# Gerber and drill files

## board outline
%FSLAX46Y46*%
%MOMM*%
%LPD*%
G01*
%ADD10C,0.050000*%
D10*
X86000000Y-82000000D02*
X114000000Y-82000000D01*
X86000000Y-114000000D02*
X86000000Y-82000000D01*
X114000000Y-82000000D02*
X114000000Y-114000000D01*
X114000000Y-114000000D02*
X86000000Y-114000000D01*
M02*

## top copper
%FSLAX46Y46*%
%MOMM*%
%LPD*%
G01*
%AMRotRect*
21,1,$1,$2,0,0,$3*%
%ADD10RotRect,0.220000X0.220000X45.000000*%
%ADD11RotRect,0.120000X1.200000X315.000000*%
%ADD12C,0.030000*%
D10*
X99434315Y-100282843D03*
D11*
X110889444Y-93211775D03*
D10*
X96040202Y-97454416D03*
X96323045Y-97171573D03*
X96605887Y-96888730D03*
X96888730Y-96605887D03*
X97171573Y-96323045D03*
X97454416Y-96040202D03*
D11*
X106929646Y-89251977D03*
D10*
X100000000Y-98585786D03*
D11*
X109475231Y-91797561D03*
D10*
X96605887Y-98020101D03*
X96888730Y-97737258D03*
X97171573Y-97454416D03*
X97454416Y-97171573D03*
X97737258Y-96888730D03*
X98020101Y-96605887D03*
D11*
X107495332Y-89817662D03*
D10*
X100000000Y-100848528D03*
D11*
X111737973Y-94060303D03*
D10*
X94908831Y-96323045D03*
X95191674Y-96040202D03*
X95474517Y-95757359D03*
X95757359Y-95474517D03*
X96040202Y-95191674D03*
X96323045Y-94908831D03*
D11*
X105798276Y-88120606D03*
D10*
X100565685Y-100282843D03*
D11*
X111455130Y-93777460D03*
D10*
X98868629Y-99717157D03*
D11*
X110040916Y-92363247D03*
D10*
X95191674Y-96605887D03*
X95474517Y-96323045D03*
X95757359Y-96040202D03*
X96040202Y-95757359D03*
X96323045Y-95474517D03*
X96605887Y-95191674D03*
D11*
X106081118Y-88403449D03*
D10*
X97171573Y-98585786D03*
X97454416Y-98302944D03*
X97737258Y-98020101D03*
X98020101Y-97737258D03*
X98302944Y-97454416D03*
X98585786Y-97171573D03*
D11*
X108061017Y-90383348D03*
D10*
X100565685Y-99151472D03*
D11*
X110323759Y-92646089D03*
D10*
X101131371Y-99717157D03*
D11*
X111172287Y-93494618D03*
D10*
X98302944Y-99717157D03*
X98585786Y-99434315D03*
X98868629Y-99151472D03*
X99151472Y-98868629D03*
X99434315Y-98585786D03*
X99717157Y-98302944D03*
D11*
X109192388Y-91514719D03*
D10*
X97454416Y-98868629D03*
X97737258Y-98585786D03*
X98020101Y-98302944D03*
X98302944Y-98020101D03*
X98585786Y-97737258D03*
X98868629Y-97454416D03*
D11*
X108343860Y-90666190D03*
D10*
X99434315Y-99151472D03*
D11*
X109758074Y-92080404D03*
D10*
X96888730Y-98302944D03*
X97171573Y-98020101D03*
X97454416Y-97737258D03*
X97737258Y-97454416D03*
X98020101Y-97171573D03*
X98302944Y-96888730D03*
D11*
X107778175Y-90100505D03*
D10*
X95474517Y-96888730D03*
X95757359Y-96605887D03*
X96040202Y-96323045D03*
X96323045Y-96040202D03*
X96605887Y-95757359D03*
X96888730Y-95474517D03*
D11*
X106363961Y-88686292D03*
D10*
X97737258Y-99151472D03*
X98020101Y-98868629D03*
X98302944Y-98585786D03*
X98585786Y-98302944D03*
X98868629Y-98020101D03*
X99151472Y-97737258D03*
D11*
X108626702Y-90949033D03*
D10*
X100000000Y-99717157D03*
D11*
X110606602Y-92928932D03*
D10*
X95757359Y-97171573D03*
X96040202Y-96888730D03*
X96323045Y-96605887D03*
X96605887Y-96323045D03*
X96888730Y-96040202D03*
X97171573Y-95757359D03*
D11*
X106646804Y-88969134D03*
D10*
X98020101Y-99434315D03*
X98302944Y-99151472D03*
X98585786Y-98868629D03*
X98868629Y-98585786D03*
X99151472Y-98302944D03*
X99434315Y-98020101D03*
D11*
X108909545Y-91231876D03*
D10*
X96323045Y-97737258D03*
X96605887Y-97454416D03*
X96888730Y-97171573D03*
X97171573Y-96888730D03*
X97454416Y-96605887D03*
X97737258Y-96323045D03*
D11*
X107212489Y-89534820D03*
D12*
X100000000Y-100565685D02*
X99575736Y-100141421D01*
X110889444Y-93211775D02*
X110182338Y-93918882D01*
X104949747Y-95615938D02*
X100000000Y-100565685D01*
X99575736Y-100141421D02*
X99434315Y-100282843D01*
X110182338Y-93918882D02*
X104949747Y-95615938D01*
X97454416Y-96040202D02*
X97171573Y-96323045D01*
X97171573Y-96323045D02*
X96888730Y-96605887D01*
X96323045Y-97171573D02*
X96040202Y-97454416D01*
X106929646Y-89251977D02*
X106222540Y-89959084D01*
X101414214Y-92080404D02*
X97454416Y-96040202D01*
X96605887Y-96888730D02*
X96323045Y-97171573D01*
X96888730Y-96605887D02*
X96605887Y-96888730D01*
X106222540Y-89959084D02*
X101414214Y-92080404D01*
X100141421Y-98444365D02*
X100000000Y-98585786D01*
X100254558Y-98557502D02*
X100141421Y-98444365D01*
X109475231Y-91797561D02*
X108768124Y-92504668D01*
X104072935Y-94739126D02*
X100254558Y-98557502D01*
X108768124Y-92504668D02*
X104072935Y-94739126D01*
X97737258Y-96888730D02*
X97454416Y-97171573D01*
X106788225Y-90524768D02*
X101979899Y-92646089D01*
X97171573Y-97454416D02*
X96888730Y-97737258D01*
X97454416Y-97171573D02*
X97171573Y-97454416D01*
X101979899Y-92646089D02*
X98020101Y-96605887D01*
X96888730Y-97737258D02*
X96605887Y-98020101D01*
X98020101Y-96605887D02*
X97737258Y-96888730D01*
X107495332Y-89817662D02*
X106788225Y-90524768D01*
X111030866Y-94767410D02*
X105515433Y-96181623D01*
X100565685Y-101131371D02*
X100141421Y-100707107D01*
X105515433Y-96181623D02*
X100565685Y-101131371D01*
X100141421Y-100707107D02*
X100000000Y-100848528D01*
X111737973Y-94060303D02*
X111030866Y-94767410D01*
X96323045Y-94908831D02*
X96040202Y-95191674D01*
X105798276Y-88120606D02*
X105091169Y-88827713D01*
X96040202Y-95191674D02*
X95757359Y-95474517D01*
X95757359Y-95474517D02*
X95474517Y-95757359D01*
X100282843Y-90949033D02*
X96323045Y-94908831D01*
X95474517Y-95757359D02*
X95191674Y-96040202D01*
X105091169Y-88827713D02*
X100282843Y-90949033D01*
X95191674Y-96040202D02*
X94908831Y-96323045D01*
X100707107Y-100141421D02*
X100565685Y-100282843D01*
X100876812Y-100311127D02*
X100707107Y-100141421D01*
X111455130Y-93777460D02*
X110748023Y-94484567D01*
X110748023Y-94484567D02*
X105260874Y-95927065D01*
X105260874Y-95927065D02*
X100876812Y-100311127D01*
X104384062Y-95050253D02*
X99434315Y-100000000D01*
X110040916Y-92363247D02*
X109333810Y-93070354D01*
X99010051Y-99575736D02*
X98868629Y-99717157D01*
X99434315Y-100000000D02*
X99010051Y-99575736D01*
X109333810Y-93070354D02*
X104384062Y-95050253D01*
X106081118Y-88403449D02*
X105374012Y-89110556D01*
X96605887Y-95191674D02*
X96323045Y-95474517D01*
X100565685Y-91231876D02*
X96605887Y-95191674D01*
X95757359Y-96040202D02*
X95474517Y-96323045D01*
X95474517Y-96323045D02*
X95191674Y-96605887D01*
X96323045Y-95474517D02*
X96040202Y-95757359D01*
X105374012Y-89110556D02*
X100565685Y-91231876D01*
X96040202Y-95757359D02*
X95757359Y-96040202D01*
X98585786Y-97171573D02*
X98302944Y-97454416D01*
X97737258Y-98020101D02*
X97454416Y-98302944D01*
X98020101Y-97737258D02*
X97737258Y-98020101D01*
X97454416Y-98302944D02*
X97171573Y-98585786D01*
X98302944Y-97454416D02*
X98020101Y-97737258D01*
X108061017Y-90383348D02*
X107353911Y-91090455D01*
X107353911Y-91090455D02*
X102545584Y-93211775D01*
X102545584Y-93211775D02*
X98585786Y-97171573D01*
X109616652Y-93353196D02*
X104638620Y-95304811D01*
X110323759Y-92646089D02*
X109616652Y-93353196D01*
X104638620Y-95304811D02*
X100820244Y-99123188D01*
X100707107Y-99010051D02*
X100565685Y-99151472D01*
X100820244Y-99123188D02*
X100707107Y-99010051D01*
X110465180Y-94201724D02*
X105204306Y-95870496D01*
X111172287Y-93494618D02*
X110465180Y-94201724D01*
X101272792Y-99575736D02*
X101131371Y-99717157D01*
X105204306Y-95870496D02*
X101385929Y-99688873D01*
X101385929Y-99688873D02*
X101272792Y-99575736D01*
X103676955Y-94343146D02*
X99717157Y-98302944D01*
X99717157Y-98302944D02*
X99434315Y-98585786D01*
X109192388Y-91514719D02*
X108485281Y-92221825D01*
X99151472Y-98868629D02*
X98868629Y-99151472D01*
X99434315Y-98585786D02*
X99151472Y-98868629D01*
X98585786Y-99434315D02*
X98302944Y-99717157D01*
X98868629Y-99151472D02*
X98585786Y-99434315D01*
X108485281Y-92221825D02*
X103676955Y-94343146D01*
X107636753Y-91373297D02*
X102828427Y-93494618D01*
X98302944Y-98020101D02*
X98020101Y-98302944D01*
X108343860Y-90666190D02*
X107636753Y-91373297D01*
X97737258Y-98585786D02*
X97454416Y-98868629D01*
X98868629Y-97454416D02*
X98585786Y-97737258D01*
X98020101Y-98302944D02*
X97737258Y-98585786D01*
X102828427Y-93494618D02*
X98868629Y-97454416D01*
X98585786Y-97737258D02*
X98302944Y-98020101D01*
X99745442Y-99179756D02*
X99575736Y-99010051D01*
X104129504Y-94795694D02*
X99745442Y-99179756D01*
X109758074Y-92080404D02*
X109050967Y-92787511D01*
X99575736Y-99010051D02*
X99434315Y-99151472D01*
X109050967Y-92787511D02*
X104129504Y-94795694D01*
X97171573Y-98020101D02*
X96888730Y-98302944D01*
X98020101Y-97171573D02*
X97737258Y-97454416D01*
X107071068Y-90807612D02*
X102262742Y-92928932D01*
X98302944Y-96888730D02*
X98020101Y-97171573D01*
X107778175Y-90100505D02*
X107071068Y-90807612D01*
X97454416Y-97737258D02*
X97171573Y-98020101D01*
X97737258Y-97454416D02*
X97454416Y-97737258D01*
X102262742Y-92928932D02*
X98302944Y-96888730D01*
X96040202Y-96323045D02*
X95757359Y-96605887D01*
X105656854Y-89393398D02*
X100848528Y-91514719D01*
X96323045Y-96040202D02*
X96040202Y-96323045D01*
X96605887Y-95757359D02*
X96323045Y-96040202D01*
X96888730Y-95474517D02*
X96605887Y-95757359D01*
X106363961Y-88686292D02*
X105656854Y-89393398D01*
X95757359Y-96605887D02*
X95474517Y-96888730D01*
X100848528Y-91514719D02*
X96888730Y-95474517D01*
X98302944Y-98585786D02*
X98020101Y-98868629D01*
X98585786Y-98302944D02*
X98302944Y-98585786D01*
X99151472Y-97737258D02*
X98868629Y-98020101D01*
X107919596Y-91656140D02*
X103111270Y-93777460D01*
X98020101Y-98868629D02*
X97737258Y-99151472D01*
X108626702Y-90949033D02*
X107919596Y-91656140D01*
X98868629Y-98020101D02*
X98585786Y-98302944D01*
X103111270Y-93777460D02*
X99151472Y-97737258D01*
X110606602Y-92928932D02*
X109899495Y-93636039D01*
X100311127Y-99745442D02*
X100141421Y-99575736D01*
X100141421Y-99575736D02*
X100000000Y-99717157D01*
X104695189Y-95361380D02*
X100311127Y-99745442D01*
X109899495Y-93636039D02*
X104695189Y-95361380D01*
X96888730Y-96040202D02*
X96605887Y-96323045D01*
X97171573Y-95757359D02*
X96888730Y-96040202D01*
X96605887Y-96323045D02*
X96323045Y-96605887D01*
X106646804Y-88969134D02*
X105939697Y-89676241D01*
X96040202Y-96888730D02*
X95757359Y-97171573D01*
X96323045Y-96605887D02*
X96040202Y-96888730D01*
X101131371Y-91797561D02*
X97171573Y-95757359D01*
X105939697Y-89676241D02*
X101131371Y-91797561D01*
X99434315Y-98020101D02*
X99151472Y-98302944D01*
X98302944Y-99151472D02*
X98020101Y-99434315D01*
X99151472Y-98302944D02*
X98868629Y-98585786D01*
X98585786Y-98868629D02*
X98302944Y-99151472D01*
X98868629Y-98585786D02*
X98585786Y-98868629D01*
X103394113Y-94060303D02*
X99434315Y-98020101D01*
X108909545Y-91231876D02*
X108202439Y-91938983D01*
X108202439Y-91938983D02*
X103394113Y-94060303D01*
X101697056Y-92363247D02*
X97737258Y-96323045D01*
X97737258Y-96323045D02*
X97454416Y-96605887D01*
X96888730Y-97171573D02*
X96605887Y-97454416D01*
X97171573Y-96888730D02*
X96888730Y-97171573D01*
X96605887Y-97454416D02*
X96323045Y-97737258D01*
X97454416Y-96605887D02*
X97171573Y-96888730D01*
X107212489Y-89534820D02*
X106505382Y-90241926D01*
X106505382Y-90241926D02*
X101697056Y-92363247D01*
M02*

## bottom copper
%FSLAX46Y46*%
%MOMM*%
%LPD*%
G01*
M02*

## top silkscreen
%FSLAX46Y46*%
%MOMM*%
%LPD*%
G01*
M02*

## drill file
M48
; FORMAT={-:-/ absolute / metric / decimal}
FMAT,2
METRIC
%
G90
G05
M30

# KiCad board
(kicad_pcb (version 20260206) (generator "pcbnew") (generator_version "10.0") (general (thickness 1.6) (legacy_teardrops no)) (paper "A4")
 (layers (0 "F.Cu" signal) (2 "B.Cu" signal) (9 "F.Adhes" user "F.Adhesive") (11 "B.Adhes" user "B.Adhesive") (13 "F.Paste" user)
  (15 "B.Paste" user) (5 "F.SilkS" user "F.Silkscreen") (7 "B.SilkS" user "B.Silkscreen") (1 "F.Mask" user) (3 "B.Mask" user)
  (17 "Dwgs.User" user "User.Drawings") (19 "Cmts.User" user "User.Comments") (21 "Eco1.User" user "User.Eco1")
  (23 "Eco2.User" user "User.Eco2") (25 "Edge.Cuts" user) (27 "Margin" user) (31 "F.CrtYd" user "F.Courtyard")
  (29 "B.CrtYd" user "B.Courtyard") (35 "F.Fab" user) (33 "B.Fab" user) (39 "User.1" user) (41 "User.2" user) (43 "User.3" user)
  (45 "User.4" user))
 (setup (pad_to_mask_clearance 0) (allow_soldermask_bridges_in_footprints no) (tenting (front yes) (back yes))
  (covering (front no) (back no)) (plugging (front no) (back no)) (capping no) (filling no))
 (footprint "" (layer "F.Cu") (at 0 0)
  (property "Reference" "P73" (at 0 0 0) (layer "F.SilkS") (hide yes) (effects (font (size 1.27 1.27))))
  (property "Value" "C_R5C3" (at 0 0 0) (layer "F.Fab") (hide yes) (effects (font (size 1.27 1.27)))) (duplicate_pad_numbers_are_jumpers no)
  (pad "1" connect rect (at 99.434315 100.282843 45) (size 0.22 0.22) (layers "F.Cu") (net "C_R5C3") (thermal_bridge_angle 45))
  (pad "2" connect rect (at 110.889444 93.211775 315) (size 0.12 1.2) (layers "F.Cu") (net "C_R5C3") (thermal_bridge_angle 45)))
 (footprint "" (layer "F.Cu") (at 0 0)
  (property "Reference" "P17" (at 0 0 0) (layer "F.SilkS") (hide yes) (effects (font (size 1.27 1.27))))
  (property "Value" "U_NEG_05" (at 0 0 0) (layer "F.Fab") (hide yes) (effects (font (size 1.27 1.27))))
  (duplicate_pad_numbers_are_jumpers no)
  (pad "1" connect rect (at 96.040202 97.454416 45) (size 0.22 0.22) (layers "F.Cu") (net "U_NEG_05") (thermal_bridge_angle 45))
  (pad "1" connect rect (at 96.323045 97.171573 45) (size 0.22 0.22) (layers "F.Cu") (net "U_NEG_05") (thermal_bridge_angle 45))
  (pad "1" connect rect (at 96.605887 96.88873 45) (size 0.22 0.22) (layers "F.Cu") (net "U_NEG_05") (thermal_bridge_angle 45))
  (pad "1" connect rect (at 96.88873 96.605887 45) (size 0.22 0.22) (layers "F.Cu") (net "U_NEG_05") (thermal_bridge_angle 45))
  (pad "1" connect rect (at 97.171573 96.323045 45) (size 0.22 0.22) (layers "F.Cu") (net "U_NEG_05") (thermal_bridge_angle 45))
  (pad "1" connect rect (at 97.454416 96.040202 45) (size 0.22 0.22) (layers "F.Cu") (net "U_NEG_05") (thermal_bridge_angle 45))
  (pad "2" connect rect (at 106.929646 89.251977 315) (size 0.12 1.2) (layers "F.Cu") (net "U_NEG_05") (thermal_bridge_angle 45)))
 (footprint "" (layer "F.Cu") (at 0 0)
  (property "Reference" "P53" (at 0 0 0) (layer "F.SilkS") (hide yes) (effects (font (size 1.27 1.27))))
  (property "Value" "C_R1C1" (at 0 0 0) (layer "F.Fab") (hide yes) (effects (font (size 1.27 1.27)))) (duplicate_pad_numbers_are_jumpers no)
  (pad "1" connect rect (at 100 98.585786 45) (size 0.22 0.22) (layers "F.Cu") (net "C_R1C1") (thermal_bridge_angle 45))
  (pad "2" connect rect (at 109.475231 91.797561 315) (size 0.12 1.2) (layers "F.Cu") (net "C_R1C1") (thermal_bridge_angle 45)))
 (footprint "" (layer "F.Cu") (at 0 0)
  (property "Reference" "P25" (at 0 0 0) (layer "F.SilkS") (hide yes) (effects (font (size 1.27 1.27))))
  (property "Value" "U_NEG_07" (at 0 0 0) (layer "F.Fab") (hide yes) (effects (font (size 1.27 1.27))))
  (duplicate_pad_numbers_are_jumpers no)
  (pad "1" connect rect (at 96.605887 98.020101 45) (size 0.22 0.22) (layers "F.Cu") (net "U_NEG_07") (thermal_bridge_angle 45))
  (pad "1" connect rect (at 96.88873 97.737258 45) (size 0.22 0.22) (layers "F.Cu") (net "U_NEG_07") (thermal_bridge_angle 45))
  (pad "1" connect rect (at 97.171573 97.454416 45) (size 0.22 0.22) (layers "F.Cu") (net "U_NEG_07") (thermal_bridge_angle 45))
  (pad "1" connect rect (at 97.454416 97.171573 45) (size 0.22 0.22) (layers "F.Cu") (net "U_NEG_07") (thermal_bridge_angle 45))
  (pad "1" connect rect (at 97.737258 96.88873 45) (size 0.22 0.22) (layers "F.Cu") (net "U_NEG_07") (thermal_bridge_angle 45))
  (pad "1" connect rect (at 98.020101 96.605887 45) (size 0.22 0.22) (layers "F.Cu") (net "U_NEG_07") (thermal_bridge_angle 45))
  (pad "2" connect rect (at 107.495332 89.817662 315) (size 0.12 1.2) (layers "F.Cu") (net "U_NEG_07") (thermal_bridge_angle 45)))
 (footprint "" (layer "F.Cu") (at 0 0)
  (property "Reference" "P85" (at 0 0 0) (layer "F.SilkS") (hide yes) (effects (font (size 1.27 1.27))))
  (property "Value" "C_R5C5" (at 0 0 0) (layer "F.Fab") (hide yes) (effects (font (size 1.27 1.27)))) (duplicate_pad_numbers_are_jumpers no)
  (pad "1" connect rect (at 100 100.848528 45) (size 0.22 0.22) (layers "F.Cu") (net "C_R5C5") (thermal_bridge_angle 45))
  (pad "2" connect rect (at 111.737973 94.060303 315) (size 0.12 1.2) (layers "F.Cu") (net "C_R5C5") (thermal_bridge_angle 45)))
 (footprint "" (layer "F.Cu") (at 0 0)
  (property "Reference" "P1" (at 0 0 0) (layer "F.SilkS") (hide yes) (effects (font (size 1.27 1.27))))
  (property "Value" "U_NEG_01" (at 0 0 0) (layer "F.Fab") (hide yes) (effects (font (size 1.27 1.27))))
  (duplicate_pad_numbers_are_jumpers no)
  (pad "1" connect rect (at 94.908831 96.323045 45) (size 0.22 0.22) (layers "F.Cu") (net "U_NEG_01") (thermal_bridge_angle 45))
  (pad "1" connect rect (at 95.191674 96.040202 45) (size 0.22 0.22) (layers "F.Cu") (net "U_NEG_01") (thermal_bridge_angle 45))
  (pad "1" connect rect (at 95.474517 95.757359 45) (size 0.22 0.22) (layers "F.Cu") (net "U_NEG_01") (thermal_bridge_angle 45))
  (pad "1" connect rect (at 95.757359 95.474517 45) (size 0.22 0.22) (layers "F.Cu") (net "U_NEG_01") (thermal_bridge_angle 45))
  (pad "1" connect rect (at 96.040202 95.191674 45) (size 0.22 0.22) (layers "F.Cu") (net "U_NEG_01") (thermal_bridge_angle 45))
  (pad "1" connect rect (at 96.323045 94.908831 45) (size 0.22 0.22) (layers "F.Cu") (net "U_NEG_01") (thermal_bridge_angle 45))
  (pad "2" connect rect (at 105.798276 88.120606 315) (size 0.12 1.2) (layers "F.Cu") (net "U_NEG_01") (thermal_bridge_angle 45)))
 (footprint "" (layer "F.Cu") (at 0 0)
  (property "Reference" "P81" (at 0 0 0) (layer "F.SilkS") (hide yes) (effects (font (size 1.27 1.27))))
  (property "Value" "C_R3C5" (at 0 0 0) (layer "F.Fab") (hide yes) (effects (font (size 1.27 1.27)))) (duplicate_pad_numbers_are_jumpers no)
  (pad "1" connect rect (at 100.565685 100.282843 45) (size 0.22 0.22) (layers "F.Cu") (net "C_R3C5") (thermal_bridge_angle 45))
  (pad "2" connect rect (at 111.45513 93.77746 315) (size 0.12 1.2) (layers "F.Cu") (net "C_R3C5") (thermal_bridge_angle 45)))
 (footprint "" (layer "F.Cu") (at 0 0)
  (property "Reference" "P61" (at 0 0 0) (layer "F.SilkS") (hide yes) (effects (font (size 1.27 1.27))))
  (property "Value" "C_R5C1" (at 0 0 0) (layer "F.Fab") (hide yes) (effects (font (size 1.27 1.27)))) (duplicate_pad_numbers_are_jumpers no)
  (pad "1" connect rect (at 98.868629 99.717157 45) (size 0.22 0.22) (layers "F.Cu") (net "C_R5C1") (thermal_bridge_angle 45))
  (pad "2" connect rect (at 110.040916 92.363247 315) (size 0.12 1.2) (layers "F.Cu") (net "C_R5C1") (thermal_bridge_angle 45)))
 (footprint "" (layer "F.Cu") (at 0 0)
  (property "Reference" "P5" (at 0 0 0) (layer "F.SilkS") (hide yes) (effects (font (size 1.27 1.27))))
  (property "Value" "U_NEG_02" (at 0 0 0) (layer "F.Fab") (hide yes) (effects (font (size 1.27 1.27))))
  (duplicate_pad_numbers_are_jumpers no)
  (pad "1" connect rect (at 95.191674 96.605887 45) (size 0.22 0.22) (layers "F.Cu") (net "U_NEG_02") (thermal_bridge_angle 45))
  (pad "1" connect rect (at 95.474517 96.323045 45) (size 0.22 0.22) (layers "F.Cu") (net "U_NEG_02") (thermal_bridge_angle 45))
  (pad "1" connect rect (at 95.757359 96.040202 45) (size 0.22 0.22) (layers "F.Cu") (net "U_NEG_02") (thermal_bridge_angle 45))
  (pad "1" connect rect (at 96.040202 95.757359 45) (size 0.22 0.22) (layers "F.Cu") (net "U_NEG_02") (thermal_bridge_angle 45))
  (pad "1" connect rect (at 96.323045 95.474517 45) (size 0.22 0.22) (layers "F.Cu") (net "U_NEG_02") (thermal_bridge_angle 45))
  (pad "1" connect rect (at 96.605887 95.191674 45) (size 0.22 0.22) (layers "F.Cu") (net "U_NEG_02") (thermal_bridge_angle 45))
  (pad "2" connect rect (at 106.081118 88.403449 315) (size 0.12 1.2) (layers "F.Cu") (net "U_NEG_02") (thermal_bridge_angle 45)))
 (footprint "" (layer "F.Cu") (at 0 0)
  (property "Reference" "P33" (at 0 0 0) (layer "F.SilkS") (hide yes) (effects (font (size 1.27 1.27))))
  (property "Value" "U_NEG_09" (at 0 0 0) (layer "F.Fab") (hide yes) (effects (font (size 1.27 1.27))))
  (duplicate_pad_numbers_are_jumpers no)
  (pad "1" connect rect (at 97.171573 98.585786 45) (size 0.22 0.22) (layers "F.Cu") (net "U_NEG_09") (thermal_bridge_angle 45))
  (pad "1" connect rect (at 97.454416 98.302944 45) (size 0.22 0.22) (layers "F.Cu") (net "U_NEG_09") (thermal_bridge_angle 45))
  (pad "1" connect rect (at 97.737258 98.020101 45) (size 0.22 0.22) (layers "F.Cu") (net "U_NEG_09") (thermal_bridge_angle 45))
  (pad "1" connect rect (at 98.020101 97.737258 45) (size 0.22 0.22) (layers "F.Cu") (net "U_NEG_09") (thermal_bridge_angle 45))
  (pad "1" connect rect (at 98.302944 97.454416 45) (size 0.22 0.22) (layers "F.Cu") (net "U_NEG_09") (thermal_bridge_angle 45))
  (pad "1" connect rect (at 98.585786 97.171573 45) (size 0.22 0.22) (layers "F.Cu") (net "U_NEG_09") (thermal_bridge_angle 45))
  (pad "2" connect rect (at 108.061017 90.383348 315) (size 0.12 1.2) (layers "F.Cu") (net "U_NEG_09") (thermal_bridge_angle 45)))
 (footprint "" (layer "F.Cu") (at 0 0)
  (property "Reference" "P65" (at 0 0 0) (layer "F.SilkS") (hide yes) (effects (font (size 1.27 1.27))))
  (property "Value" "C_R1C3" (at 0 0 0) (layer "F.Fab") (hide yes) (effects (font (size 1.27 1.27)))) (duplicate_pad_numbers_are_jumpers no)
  (pad "1" connect rect (at 100.565685 99.151472 45) (size 0.22 0.22) (layers "F.Cu") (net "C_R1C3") (thermal_bridge_angle 45))
  (pad "2" connect rect (at 110.323759 92.646089 315) (size 0.12 1.2) (layers "F.Cu") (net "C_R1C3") (thermal_bridge_angle 45)))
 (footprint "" (layer "F.Cu") (at 0 0)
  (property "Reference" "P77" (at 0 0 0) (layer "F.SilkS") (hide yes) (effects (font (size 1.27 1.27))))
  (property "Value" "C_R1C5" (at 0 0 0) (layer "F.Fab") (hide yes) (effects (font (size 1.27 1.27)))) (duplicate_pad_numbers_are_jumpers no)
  (pad "1" connect rect (at 101.131371 99.717157 45) (size 0.22 0.22) (layers "F.Cu") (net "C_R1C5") (thermal_bridge_angle 45))
  (pad "2" connect rect (at 111.172287 93.494618 315) (size 0.12 1.2) (layers "F.Cu") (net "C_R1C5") (thermal_bridge_angle 45)))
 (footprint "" (layer "F.Cu") (at 0 0)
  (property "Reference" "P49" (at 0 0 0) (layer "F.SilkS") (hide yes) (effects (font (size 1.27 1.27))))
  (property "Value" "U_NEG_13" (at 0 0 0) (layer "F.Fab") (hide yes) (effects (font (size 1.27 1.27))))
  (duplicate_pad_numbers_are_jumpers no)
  (pad "1" connect rect (at 98.302944 99.717157 45) (size 0.22 0.22) (layers "F.Cu") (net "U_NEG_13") (thermal_bridge_angle 45))
  (pad "1" connect rect (at 98.585786 99.434315 45) (size 0.22 0.22) (layers "F.Cu") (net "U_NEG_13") (thermal_bridge_angle 45))
  (pad "1" connect rect (at 98.868629 99.151472 45) (size 0.22 0.22) (layers "F.Cu") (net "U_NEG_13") (thermal_bridge_angle 45))
  (pad "1" connect rect (at 99.151472 98.868629 45) (size 0.22 0.22) (layers "F.Cu") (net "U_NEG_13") (thermal_bridge_angle 45))
  (pad "1" connect rect (at 99.434315 98.585786 45) (size 0.22 0.22) (layers "F.Cu") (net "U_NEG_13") (thermal_bridge_angle 45))
  (pad "1" connect rect (at 99.717157 98.302944 45) (size 0.22 0.22) (layers "F.Cu") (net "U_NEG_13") (thermal_bridge_angle 45))
  (pad "2" connect rect (at 109.192388 91.514719 315) (size 0.12 1.2) (layers "F.Cu") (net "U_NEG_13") (thermal_bridge_angle 45)))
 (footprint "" (layer "F.Cu") (at 0 0)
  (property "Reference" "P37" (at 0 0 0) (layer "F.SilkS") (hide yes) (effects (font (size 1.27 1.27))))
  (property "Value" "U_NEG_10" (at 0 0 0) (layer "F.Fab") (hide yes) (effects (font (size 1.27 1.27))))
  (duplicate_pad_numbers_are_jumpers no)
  (pad "1" connect rect (at 97.454416 98.868629 45) (size 0.22 0.22) (layers "F.Cu") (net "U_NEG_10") (thermal_bridge_angle 45))
  (pad "1" connect rect (at 97.737258 98.585786 45) (size 0.22 0.22) (layers "F.Cu") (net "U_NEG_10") (thermal_bridge_angle 45))
  (pad "1" connect rect (at 98.020101 98.302944 45) (size 0.22 0.22) (layers "F.Cu") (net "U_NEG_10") (thermal_bridge_angle 45))
  (pad "1" connect rect (at 98.302944 98.020101 45) (size 0.22 0.22) (layers "F.Cu") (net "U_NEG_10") (thermal_bridge_angle 45))
  (pad "1" connect rect (at 98.585786 97.737258 45) (size 0.22 0.22) (layers "F.Cu") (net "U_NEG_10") (thermal_bridge_angle 45))
  (pad "1" connect rect (at 98.868629 97.454416 45) (size 0.22 0.22) (layers "F.Cu") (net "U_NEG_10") (thermal_bridge_angle 45))
  (pad "2" connect rect (at 108.34386 90.66619 315) (size 0.12 1.2) (layers "F.Cu") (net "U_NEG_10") (thermal_bridge_angle 45)))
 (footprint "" (layer "F.Cu") (at 0 0)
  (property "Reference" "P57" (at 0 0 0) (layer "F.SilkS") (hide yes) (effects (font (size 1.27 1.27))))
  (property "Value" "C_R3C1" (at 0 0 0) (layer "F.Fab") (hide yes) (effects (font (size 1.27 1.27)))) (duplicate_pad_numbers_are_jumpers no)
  (pad "1" connect rect (at 99.434315 99.151472 45) (size 0.22 0.22) (layers "F.Cu") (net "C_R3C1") (thermal_bridge_angle 45))
  (pad "2" connect rect (at 109.758074 92.080404 315) (size 0.12 1.2) (layers "F.Cu") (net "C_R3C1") (thermal_bridge_angle 45)))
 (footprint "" (layer "F.Cu") (at 0 0)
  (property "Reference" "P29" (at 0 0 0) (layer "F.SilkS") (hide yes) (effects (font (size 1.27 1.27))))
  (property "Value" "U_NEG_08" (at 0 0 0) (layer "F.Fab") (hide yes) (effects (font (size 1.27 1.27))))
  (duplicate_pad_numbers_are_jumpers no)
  (pad "1" connect rect (at 96.88873 98.302944 45) (size 0.22 0.22) (layers "F.Cu") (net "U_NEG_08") (thermal_bridge_angle 45))
  (pad "1" connect rect (at 97.171573 98.020101 45) (size 0.22 0.22) (layers "F.Cu") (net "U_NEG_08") (thermal_bridge_angle 45))
  (pad "1" connect rect (at 97.454416 97.737258 45) (size 0.22 0.22) (layers "F.Cu") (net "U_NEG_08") (thermal_bridge_angle 45))
  (pad "1" connect rect (at 97.737258 97.454416 45) (size 0.22 0.22) (layers "F.Cu") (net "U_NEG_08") (thermal_bridge_angle 45))
  (pad "1" connect rect (at 98.020101 97.171573 45) (size 0.22 0.22) (layers "F.Cu") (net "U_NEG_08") (thermal_bridge_angle 45))
  (pad "1" connect rect (at 98.302944 96.88873 45) (size 0.22 0.22) (layers "F.Cu") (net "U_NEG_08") (thermal_bridge_angle 45))
  (pad "2" connect rect (at 107.778175 90.100505 315) (size 0.12 1.2) (layers "F.Cu") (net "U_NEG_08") (thermal_bridge_angle 45)))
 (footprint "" (layer "F.Cu") (at 0 0)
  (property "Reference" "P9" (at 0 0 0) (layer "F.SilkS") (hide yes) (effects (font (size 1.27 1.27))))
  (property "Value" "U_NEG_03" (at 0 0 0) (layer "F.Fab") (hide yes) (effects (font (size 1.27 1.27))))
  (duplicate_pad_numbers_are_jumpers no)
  (pad "1" connect rect (at 95.474517 96.88873 45) (size 0.22 0.22) (layers "F.Cu") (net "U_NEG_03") (thermal_bridge_angle 45))
  (pad "1" connect rect (at 95.757359 96.605887 45) (size 0.22 0.22) (layers "F.Cu") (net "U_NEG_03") (thermal_bridge_angle 45))
  (pad "1" connect rect (at 96.040202 96.323045 45) (size 0.22 0.22) (layers "F.Cu") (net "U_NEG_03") (thermal_bridge_angle 45))
  (pad "1" connect rect (at 96.323045 96.040202 45) (size 0.22 0.22) (layers "F.Cu") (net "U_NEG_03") (thermal_bridge_angle 45))
  (pad "1" connect rect (at 96.605887 95.757359 45) (size 0.22 0.22) (layers "F.Cu") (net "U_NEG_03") (thermal_bridge_angle 45))
  (pad "1" connect rect (at 96.88873 95.474517 45) (size 0.22 0.22) (layers "F.Cu") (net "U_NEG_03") (thermal_bridge_angle 45))
  (pad "2" connect rect (at 106.363961 88.686292 315) (size 0.12 1.2) (layers "F.Cu") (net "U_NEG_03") (thermal_bridge_angle 45)))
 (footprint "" (layer "F.Cu") (at 0 0)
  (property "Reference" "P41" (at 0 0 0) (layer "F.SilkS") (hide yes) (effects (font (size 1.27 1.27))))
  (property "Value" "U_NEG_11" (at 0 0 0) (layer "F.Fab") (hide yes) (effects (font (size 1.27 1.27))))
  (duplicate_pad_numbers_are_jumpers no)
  (pad "1" connect rect (at 97.737258 99.151472 45) (size 0.22 0.22) (layers "F.Cu") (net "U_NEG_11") (thermal_bridge_angle 45))
  (pad "1" connect rect (at 98.020101 98.868629 45) (size 0.22 0.22) (layers "F.Cu") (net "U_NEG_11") (thermal_bridge_angle 45))
  (pad "1" connect rect (at 98.302944 98.585786 45) (size 0.22 0.22) (layers "F.Cu") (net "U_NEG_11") (thermal_bridge_angle 45))
  (pad "1" connect rect (at 98.585786 98.302944 45) (size 0.22 0.22) (layers "F.Cu") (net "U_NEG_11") (thermal_bridge_angle 45))
  (pad "1" connect rect (at 98.868629 98.020101 45) (size 0.22 0.22) (layers "F.Cu") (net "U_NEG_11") (thermal_bridge_angle 45))
  (pad "1" connect rect (at 99.151472 97.737258 45) (size 0.22 0.22) (layers "F.Cu") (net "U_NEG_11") (thermal_bridge_angle 45))
  (pad "2" connect rect (at 108.626702 90.949033 315) (size 0.12 1.2) (layers "F.Cu") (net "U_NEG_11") (thermal_bridge_angle 45)))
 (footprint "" (layer "F.Cu") (at 0 0)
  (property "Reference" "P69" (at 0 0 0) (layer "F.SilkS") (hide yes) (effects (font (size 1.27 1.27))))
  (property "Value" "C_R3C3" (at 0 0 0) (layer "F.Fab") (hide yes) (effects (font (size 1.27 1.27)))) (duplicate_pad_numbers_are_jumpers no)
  (pad "1" connect rect (at 100 99.717157 45) (size 0.22 0.22) (layers "F.Cu") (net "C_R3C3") (thermal_bridge_angle 45))
  (pad "2" connect rect (at 110.606602 92.928932 315) (size 0.12 1.2) (layers "F.Cu") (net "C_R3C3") (thermal_bridge_angle 45)))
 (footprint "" (layer "F.Cu") (at 0 0)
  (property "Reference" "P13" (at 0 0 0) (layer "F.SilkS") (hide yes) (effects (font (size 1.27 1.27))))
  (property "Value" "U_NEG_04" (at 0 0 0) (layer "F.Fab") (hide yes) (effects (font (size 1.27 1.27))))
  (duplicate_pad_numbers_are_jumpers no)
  (pad "1" connect rect (at 95.757359 97.171573 45) (size 0.22 0.22) (layers "F.Cu") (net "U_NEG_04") (thermal_bridge_angle 45))
  (pad "1" connect rect (at 96.040202 96.88873 45) (size 0.22 0.22) (layers "F.Cu") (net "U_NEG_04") (thermal_bridge_angle 45))
  (pad "1" connect rect (at 96.323045 96.605887 45) (size 0.22 0.22) (layers "F.Cu") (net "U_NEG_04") (thermal_bridge_angle 45))
  (pad "1" connect rect (at 96.605887 96.323045 45) (size 0.22 0.22) (layers "F.Cu") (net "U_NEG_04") (thermal_bridge_angle 45))
  (pad "1" connect rect (at 96.88873 96.040202 45) (size 0.22 0.22) (layers "F.Cu") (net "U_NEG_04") (thermal_bridge_angle 45))
  (pad "1" connect rect (at 97.171573 95.757359 45) (size 0.22 0.22) (layers "F.Cu") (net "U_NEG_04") (thermal_bridge_angle 45))
  (pad "2" connect rect (at 106.646804 88.969134 315) (size 0.12 1.2) (layers "F.Cu") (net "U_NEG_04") (thermal_bridge_angle 45)))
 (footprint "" (layer "F.Cu") (at 0 0)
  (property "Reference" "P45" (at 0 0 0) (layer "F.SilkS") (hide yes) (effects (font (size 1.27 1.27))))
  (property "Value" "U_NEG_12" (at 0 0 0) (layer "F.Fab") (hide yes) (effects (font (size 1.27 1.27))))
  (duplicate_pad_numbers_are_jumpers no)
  (pad "1" connect rect (at 98.020101 99.434315 45) (size 0.22 0.22) (layers "F.Cu") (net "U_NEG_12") (thermal_bridge_angle 45))
  (pad "1" connect rect (at 98.302944 99.151472 45) (size 0.22 0.22) (layers "F.Cu") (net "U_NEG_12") (thermal_bridge_angle 45))
  (pad "1" connect rect (at 98.585786 98.868629 45) (size 0.22 0.22) (layers "F.Cu") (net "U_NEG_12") (thermal_bridge_angle 45))
  (pad "1" connect rect (at 98.868629 98.585786 45) (size 0.22 0.22) (layers "F.Cu") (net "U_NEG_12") (thermal_bridge_angle 45))
  (pad "1" connect rect (at 99.151472 98.302944 45) (size 0.22 0.22) (layers "F.Cu") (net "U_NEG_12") (thermal_bridge_angle 45))
  (pad "1" connect rect (at 99.434315 98.020101 45) (size 0.22 0.22) (layers "F.Cu") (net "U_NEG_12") (thermal_bridge_angle 45))
  (pad "2" connect rect (at 108.909545 91.231876 315) (size 0.12 1.2) (layers "F.Cu") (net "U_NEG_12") (thermal_bridge_angle 45)))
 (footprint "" (layer "F.Cu") (at 0 0)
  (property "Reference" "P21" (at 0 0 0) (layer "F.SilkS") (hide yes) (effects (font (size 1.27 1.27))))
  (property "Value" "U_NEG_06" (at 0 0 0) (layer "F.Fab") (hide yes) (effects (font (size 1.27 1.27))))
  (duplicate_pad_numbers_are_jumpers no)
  (pad "1" connect rect (at 96.323045 97.737258 45) (size 0.22 0.22) (layers "F.Cu") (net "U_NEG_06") (thermal_bridge_angle 45))
  (pad "1" connect rect (at 96.605887 97.454416 45) (size 0.22 0.22) (layers "F.Cu") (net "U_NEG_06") (thermal_bridge_angle 45))
  (pad "1" connect rect (at 96.88873 97.171573 45) (size 0.22 0.22) (layers "F.Cu") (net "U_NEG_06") (thermal_bridge_angle 45))
  (pad "1" connect rect (at 97.171573 96.88873 45) (size 0.22 0.22) (layers "F.Cu") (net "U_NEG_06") (thermal_bridge_angle 45))
  (pad "1" connect rect (at 97.454416 96.605887 45) (size 0.22 0.22) (layers "F.Cu") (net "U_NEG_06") (thermal_bridge_angle 45))
  (pad "1" connect rect (at 97.737258 96.323045 45) (size 0.22 0.22) (layers "F.Cu") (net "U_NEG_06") (thermal_bridge_angle 45))
  (pad "2" connect rect (at 107.212489 89.53482 315) (size 0.12 1.2) (layers "F.Cu") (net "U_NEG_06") (thermal_bridge_angle 45)))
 (gr_line (start 86 82) (end 114 82) (stroke (width 0.05) (type default)) (layer "Edge.Cuts"))
 (gr_line (start 86 114) (end 86 82) (stroke (width 0.05) (type default)) (layer "Edge.Cuts"))
 (gr_line (start 114 82) (end 114 114) (stroke (width 0.05) (type default)) (layer "Edge.Cuts"))
 (gr_line (start 114 114) (end 86 114) (stroke (width 0.05) (type default)) (layer "Edge.Cuts"))
 (segment (start 100 100.565685) (end 99.575736 100.141421) (width 0.03) (layer "F.Cu") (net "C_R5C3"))
 (segment (start 110.889444 93.211775) (end 110.182338 93.918882) (width 0.03) (layer "F.Cu") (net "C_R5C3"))
 (segment (start 104.949747 95.615938) (end 100 100.565685) (width 0.03) (layer "F.Cu") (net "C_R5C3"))
 (segment (start 99.575736 100.141421) (end 99.434315 100.282843) (width 0.03) (layer "F.Cu") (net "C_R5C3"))
 (segment (start 110.182338 93.918882) (end 104.949747 95.615938) (width 0.03) (layer "F.Cu") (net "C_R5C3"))
 (segment (start 97.454416 96.040202) (end 97.171573 96.323045) (width 0.03) (layer "F.Cu") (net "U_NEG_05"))
 (segment (start 97.171573 96.323045) (end 96.88873 96.605887) (width 0.03) (layer "F.Cu") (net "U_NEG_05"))
 (segment (start 96.323045 97.171573) (end 96.040202 97.454416) (width 0.03) (layer "F.Cu") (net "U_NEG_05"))
 (segment (start 106.929646 89.251977) (end 106.22254 89.959084) (width 0.03) (layer "F.Cu") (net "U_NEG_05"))
 (segment (start 101.414214 92.080404) (end 97.454416 96.040202) (width 0.03) (layer "F.Cu") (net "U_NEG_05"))
 (segment (start 96.605887 96.88873) (end 96.323045 97.171573) (width 0.03) (layer "F.Cu") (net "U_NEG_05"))
 (segment (start 96.88873 96.605887) (end 96.605887 96.88873) (width 0.03) (layer "F.Cu") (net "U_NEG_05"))
 (segment (start 106.22254 89.959084) (end 101.414214 92.080404) (width 0.03) (layer "F.Cu") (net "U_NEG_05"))
 (segment (start 100.141421 98.444365) (end 100 98.585786) (width 0.03) (layer "F.Cu") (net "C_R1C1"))
 (segment (start 100.254558 98.557502) (end 100.141421 98.444365) (width 0.03) (layer "F.Cu") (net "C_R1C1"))
 (segment (start 109.475231 91.797561) (end 108.768124 92.504668) (width 0.03) (layer "F.Cu") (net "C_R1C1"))
 (segment (start 104.072935 94.739126) (end 100.254558 98.557502) (width 0.03) (layer "F.Cu") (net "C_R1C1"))
 (segment (start 108.768124 92.504668) (end 104.072935 94.739126) (width 0.03) (layer "F.Cu") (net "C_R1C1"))
 (segment (start 97.737258 96.88873) (end 97.454416 97.171573) (width 0.03) (layer "F.Cu") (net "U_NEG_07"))
 (segment (start 106.788225 90.524768) (end 101.979899 92.646089) (width 0.03) (layer "F.Cu") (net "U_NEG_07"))
 (segment (start 97.171573 97.454416) (end 96.88873 97.737258) (width 0.03) (layer "F.Cu") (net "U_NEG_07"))
 (segment (start 97.454416 97.171573) (end 97.171573 97.454416) (width 0.03) (layer "F.Cu") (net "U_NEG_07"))
 (segment (start 101.979899 92.646089) (end 98.020101 96.605887) (width 0.03) (layer "F.Cu") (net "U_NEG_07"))
 (segment (start 96.88873 97.737258) (end 96.605887 98.020101) (width 0.03) (layer "F.Cu") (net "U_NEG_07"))
 (segment (start 98.020101 96.605887) (end 97.737258 96.88873) (width 0.03) (layer "F.Cu") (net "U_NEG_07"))
 (segment (start 107.495332 89.817662) (end 106.788225 90.524768) (width 0.03) (layer "F.Cu") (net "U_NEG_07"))
 (segment (start 111.030866 94.76741) (end 105.515433 96.181623) (width 0.03) (layer "F.Cu") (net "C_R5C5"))
 (segment (start 100.565685 101.131371) (end 100.141421 100.707107) (width 0.03) (layer "F.Cu") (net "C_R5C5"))
 (segment (start 105.515433 96.181623) (end 100.565685 101.131371) (width 0.03) (layer "F.Cu") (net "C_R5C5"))
 (segment (start 100.141421 100.707107) (end 100 100.848528) (width 0.03) (layer "F.Cu") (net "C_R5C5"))
 (segment (start 111.737973 94.060303) (end 111.030866 94.76741) (width 0.03) (layer "F.Cu") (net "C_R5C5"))
 (segment (start 96.323045 94.908831) (end 96.040202 95.191674) (width 0.03) (layer "F.Cu") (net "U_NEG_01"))
 (segment (start 105.798276 88.120606) (end 105.091169 88.827713) (width 0.03) (layer "F.Cu") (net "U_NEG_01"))
 (segment (start 96.040202 95.191674) (end 95.757359 95.474517) (width 0.03) (layer "F.Cu") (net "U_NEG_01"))
 (segment (start 95.757359 95.474517) (end 95.474517 95.757359) (width 0.03) (layer "F.Cu") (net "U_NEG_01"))
 (segment (start 100.282843 90.949033) (end 96.323045 94.908831) (width 0.03) (layer "F.Cu") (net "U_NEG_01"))
 (segment (start 95.474517 95.757359) (end 95.191674 96.040202) (width 0.03) (layer "F.Cu") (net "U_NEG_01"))
 (segment (start 105.091169 88.827713) (end 100.282843 90.949033) (width 0.03) (layer "F.Cu") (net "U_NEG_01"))
 (segment (start 95.191674 96.040202) (end 94.908831 96.323045) (width 0.03) (layer "F.Cu") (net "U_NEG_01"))
 (segment (start 100.707107 100.141421) (end 100.565685 100.282843) (width 0.03) (layer "F.Cu") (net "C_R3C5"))
 (segment (start 100.876812 100.311127) (end 100.707107 100.141421) (width 0.03) (layer "F.Cu") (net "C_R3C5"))
 (segment (start 111.45513 93.77746) (end 110.748023 94.484567) (width 0.03) (layer "F.Cu") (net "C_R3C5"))
 (segment (start 110.748023 94.484567) (end 105.260874 95.927065) (width 0.03) (layer "F.Cu") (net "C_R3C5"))
 (segment (start 105.260874 95.927065) (end 100.876812 100.311127) (width 0.03) (layer "F.Cu") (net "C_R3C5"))
 (segment (start 104.384062 95.050253) (end 99.434315 100) (width 0.03) (layer "F.Cu") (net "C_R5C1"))
 (segment (start 110.040916 92.363247) (end 109.33381 93.070354) (width 0.03) (layer "F.Cu") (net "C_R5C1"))
 (segment (start 99.010051 99.575736) (end 98.868629 99.717157) (width 0.03) (layer "F.Cu") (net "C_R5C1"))
 (segment (start 99.434315 100) (end 99.010051 99.575736) (width 0.03) (layer "F.Cu") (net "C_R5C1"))
 (segment (start 109.33381 93.070354) (end 104.384062 95.050253) (width 0.03) (layer "F.Cu") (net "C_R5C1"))
 (segment (start 106.081118 88.403449) (end 105.374012 89.110556) (width 0.03) (layer "F.Cu") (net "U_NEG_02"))
 (segment (start 96.605887 95.191674) (end 96.323045 95.474517) (width 0.03) (layer "F.Cu") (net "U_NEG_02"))
 (segment (start 100.565685 91.231876) (end 96.605887 95.191674) (width 0.03) (layer "F.Cu") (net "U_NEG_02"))
 (segment (start 95.757359 96.040202) (end 95.474517 96.323045) (width 0.03) (layer "F.Cu") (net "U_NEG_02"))
 (segment (start 95.474517 96.323045) (end 95.191674 96.605887) (width 0.03) (layer "F.Cu") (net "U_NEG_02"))
 (segment (start 96.323045 95.474517) (end 96.040202 95.757359) (width 0.03) (layer "F.Cu") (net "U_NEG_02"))
 (segment (start 105.374012 89.110556) (end 100.565685 91.231876) (width 0.03) (layer "F.Cu") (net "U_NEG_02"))
 (segment (start 96.040202 95.757359) (end 95.757359 96.040202) (width 0.03) (layer "F.Cu") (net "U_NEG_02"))
 (segment (start 98.585786 97.171573) (end 98.302944 97.454416) (width 0.03) (layer "F.Cu") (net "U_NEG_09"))
 (segment (start 97.737258 98.020101) (end 97.454416 98.302944) (width 0.03) (layer "F.Cu") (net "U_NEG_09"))
 (segment (start 98.020101 97.737258) (end 97.737258 98.020101) (width 0.03) (layer "F.Cu") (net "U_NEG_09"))
 (segment (start 97.454416 98.302944) (end 97.171573 98.585786) (width 0.03) (layer "F.Cu") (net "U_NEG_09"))
 (segment (start 98.302944 97.454416) (end 98.020101 97.737258) (width 0.03) (layer "F.Cu") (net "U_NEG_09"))
 (segment (start 108.061017 90.383348) (end 107.353911 91.090455) (width 0.03) (layer "F.Cu") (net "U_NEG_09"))
 (segment (start 107.353911 91.090455) (end 102.545584 93.211775) (width 0.03) (layer "F.Cu") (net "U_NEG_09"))
 (segment (start 102.545584 93.211775) (end 98.585786 97.171573) (width 0.03) (layer "F.Cu") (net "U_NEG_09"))
 (segment (start 109.616652 93.353196) (end 104.63862 95.304811) (width 0.03) (layer "F.Cu") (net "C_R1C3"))
 (segment (start 110.323759 92.646089) (end 109.616652 93.353196) (width 0.03) (layer "F.Cu") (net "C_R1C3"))
 (segment (start 104.63862 95.304811) (end 100.820244 99.123188) (width 0.03) (layer "F.Cu") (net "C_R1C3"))
 (segment (start 100.707107 99.010051) (end 100.565685 99.151472) (width 0.03) (layer "F.Cu") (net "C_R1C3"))
 (segment (start 100.820244 99.123188) (end 100.707107 99.010051) (width 0.03) (layer "F.Cu") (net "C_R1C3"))
 (segment (start 110.46518 94.201724) (end 105.204306 95.870496) (width 0.03) (layer "F.Cu") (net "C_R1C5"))
 (segment (start 111.172287 93.494618) (end 110.46518 94.201724) (width 0.03) (layer "F.Cu") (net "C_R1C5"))
 (segment (start 101.272792 99.575736) (end 101.131371 99.717157) (width 0.03) (layer "F.Cu") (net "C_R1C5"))
 (segment (start 105.204306 95.870496) (end 101.385929 99.688873) (width 0.03) (layer "F.Cu") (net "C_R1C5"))
 (segment (start 101.385929 99.688873) (end 101.272792 99.575736) (width 0.03) (layer "F.Cu") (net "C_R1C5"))
 (segment (start 103.676955 94.343146) (end 99.717157 98.302944) (width 0.03) (layer "F.Cu") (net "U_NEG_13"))
 (segment (start 99.717157 98.302944) (end 99.434315 98.585786) (width 0.03) (layer "F.Cu") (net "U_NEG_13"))
 (segment (start 109.192388 91.514719) (end 108.485281 92.221825) (width 0.03) (layer "F.Cu") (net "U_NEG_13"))
 (segment (start 99.151472 98.868629) (end 98.868629 99.151472) (width 0.03) (layer "F.Cu") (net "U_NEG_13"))
 (segment (start 99.434315 98.585786) (end 99.151472 98.868629) (width 0.03) (layer "F.Cu") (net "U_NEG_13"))
 (segment (start 98.585786 99.434315) (end 98.302944 99.717157) (width 0.03) (layer "F.Cu") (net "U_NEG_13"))
 (segment (start 98.868629 99.151472) (end 98.585786 99.434315) (width 0.03) (layer "F.Cu") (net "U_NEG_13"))
 (segment (start 108.485281 92.221825) (end 103.676955 94.343146) (width 0.03) (layer "F.Cu") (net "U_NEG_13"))
 (segment (start 107.636753 91.373297) (end 102.828427 93.494618) (width 0.03) (layer "F.Cu") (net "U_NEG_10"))
 (segment (start 98.302944 98.020101) (end 98.020101 98.302944) (width 0.03) (layer "F.Cu") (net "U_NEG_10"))
 (segment (start 108.34386 90.66619) (end 107.636753 91.373297) (width 0.03) (layer "F.Cu") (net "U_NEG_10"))
 (segment (start 97.737258 98.585786) (end 97.454416 98.868629) (width 0.03) (layer "F.Cu") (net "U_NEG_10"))
 (segment (start 98.868629 97.454416) (end 98.585786 97.737258) (width 0.03) (layer "F.Cu") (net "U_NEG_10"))
 (segment (start 98.020101 98.302944) (end 97.737258 98.585786) (width 0.03) (layer "F.Cu") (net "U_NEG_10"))
 (segment (start 102.828427 93.494618) (end 98.868629 97.454416) (width 0.03) (layer "F.Cu") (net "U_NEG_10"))
 (segment (start 98.585786 97.737258) (end 98.302944 98.020101) (width 0.03) (layer "F.Cu") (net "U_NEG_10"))
 (segment (start 99.745442 99.179756) (end 99.575736 99.010051) (width 0.03) (layer "F.Cu") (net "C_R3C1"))
 (segment (start 104.129504 94.795694) (end 99.745442 99.179756) (width 0.03) (layer "F.Cu") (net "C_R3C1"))
 (segment (start 109.758074 92.080404) (end 109.050967 92.787511) (width 0.03) (layer "F.Cu") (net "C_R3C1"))
 (segment (start 99.575736 99.010051) (end 99.434315 99.151472) (width 0.03) (layer "F.Cu") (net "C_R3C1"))
 (segment (start 109.050967 92.787511) (end 104.129504 94.795694) (width 0.03) (layer "F.Cu") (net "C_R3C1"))
 (segment (start 97.171573 98.020101) (end 96.88873 98.302944) (width 0.03) (layer "F.Cu") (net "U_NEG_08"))
 (segment (start 98.020101 97.171573) (end 97.737258 97.454416) (width 0.03) (layer "F.Cu") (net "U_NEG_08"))
 (segment (start 107.071068 90.807612) (end 102.262742 92.928932) (width 0.03) (layer "F.Cu") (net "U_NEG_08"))
 (segment (start 98.302944 96.88873) (end 98.020101 97.171573) (width 0.03) (layer "F.Cu") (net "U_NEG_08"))
 (segment (start 107.778175 90.100505) (end 107.071068 90.807612) (width 0.03) (layer "F.Cu") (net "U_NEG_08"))
 (segment (start 97.454416 97.737258) (end 97.171573 98.020101) (width 0.03) (layer "F.Cu") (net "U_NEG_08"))
 (segment (start 97.737258 97.454416) (end 97.454416 97.737258) (width 0.03) (layer "F.Cu") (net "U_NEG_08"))
 (segment (start 102.262742 92.928932) (end 98.302944 96.88873) (width 0.03) (layer "F.Cu") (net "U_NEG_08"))
 (segment (start 96.040202 96.323045) (end 95.757359 96.605887) (width 0.03) (layer "F.Cu") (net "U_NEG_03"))
 (segment (start 105.656854 89.393398) (end 100.848528 91.514719) (width 0.03) (layer "F.Cu") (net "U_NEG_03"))
 (segment (start 96.323045 96.040202) (end 96.040202 96.323045) (width 0.03) (layer "F.Cu") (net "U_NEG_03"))
 (segment (start 96.605887 95.757359) (end 96.323045 96.040202) (width 0.03) (layer "F.Cu") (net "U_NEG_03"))
 (segment (start 96.88873 95.474517) (end 96.605887 95.757359) (width 0.03) (layer "F.Cu") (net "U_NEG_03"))
 (segment (start 106.363961 88.686292) (end 105.656854 89.393398) (width 0.03) (layer "F.Cu") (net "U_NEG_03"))
 (segment (start 95.757359 96.605887) (end 95.474517 96.88873) (width 0.03) (layer "F.Cu") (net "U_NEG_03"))
 (segment (start 100.848528 91.514719) (end 96.88873 95.474517) (width 0.03) (layer "F.Cu") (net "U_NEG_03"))
 (segment (start 98.302944 98.585786) (end 98.020101 98.868629) (width 0.03) (layer "F.Cu") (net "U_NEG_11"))
 (segment (start 98.585786 98.302944) (end 98.302944 98.585786) (width 0.03) (layer "F.Cu") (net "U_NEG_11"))
 (segment (start 99.151472 97.737258) (end 98.868629 98.020101) (width 0.03) (layer "F.Cu") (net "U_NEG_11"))
 (segment (start 107.919596 91.65614) (end 103.11127 93.77746) (width 0.03) (layer "F.Cu") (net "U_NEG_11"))
 (segment (start 98.020101 98.868629) (end 97.737258 99.151472) (width 0.03) (layer "F.Cu") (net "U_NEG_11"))
 (segment (start 108.626702 90.949033) (end 107.919596 91.65614) (width 0.03) (layer "F.Cu") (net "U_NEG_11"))
 (segment (start 98.868629 98.020101) (end 98.585786 98.302944) (width 0.03) (layer "F.Cu") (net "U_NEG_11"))
 (segment (start 103.11127 93.77746) (end 99.151472 97.737258) (width 0.03) (layer "F.Cu") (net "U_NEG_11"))
 (segment (start 110.606602 92.928932) (end 109.899495 93.636039) (width 0.03) (layer "F.Cu") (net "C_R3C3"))
 (segment (start 100.311127 99.745442) (end 100.141421 99.575736) (width 0.03) (layer "F.Cu") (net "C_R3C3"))
 (segment (start 100.141421 99.575736) (end 100 99.717157) (width 0.03) (layer "F.Cu") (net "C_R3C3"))
 (segment (start 104.695189 95.36138) (end 100.311127 99.745442) (width 0.03) (layer "F.Cu") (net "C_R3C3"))
 (segment (start 109.899495 93.636039) (end 104.695189 95.36138) (width 0.03) (layer "F.Cu") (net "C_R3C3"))
 (segment (start 96.88873 96.040202) (end 96.605887 96.323045) (width 0.03) (layer "F.Cu") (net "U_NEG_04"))
 (segment (start 97.171573 95.757359) (end 96.88873 96.040202) (width 0.03) (layer "F.Cu") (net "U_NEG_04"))
 (segment (start 96.605887 96.323045) (end 96.323045 96.605887) (width 0.03) (layer "F.Cu") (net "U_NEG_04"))
 (segment (start 106.646804 88.969134) (end 105.939697 89.676241) (width 0.03) (layer "F.Cu") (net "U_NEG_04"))
 (segment (start 96.040202 96.88873) (end 95.757359 97.171573) (width 0.03) (layer "F.Cu") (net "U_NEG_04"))
 (segment (start 96.323045 96.605887) (end 96.040202 96.88873) (width 0.03) (layer "F.Cu") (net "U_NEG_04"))
 (segment (start 101.131371 91.797561) (end 97.171573 95.757359) (width 0.03) (layer "F.Cu") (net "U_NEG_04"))
 (segment (start 105.939697 89.676241) (end 101.131371 91.797561) (width 0.03) (layer "F.Cu") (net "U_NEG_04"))
 (segment (start 99.434315 98.020101) (end 99.151472 98.302944) (width 0.03) (layer "F.Cu") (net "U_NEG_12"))
 (segment (start 98.302944 99.151472) (end 98.020101 99.434315) (width 0.03) (layer "F.Cu") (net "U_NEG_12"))
 (segment (start 99.151472 98.302944) (end 98.868629 98.585786) (width 0.03) (layer "F.Cu") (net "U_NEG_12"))
 (segment (start 98.585786 98.868629) (end 98.302944 99.151472) (width 0.03) (layer "F.Cu") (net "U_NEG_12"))
 (segment (start 98.868629 98.585786) (end 98.585786 98.868629) (width 0.03) (layer "F.Cu") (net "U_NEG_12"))
 (segment (start 103.394113 94.060303) (end 99.434315 98.020101) (width 0.03) (layer "F.Cu") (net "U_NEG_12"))
 (segment (start 108.909545 91.231876) (end 108.202439 91.938983) (width 0.03) (layer "F.Cu") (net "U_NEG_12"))
 (segment (start 108.202439 91.938983) (end 103.394113 94.060303) (width 0.03) (layer "F.Cu") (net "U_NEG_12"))
 (segment (start 101.697056 92.363247) (end 97.737258 96.323045) (width 0.03) (layer "F.Cu") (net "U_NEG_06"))
 (segment (start 97.737258 96.323045) (end 97.454416 96.605887) (width 0.03) (layer "F.Cu") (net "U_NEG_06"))
 (segment (start 96.88873 97.171573) (end 96.605887 97.454416) (width 0.03) (layer "F.Cu") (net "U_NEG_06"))
 (segment (start 97.171573 96.88873) (end 96.88873 97.171573) (width 0.03) (layer "F.Cu") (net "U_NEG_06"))
 (segment (start 96.605887 97.454416) (end 96.323045 97.737258) (width 0.03) (layer "F.Cu") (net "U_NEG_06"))
 (segment (start 97.454416 96.605887) (end 97.171573 96.88873) (width 0.03) (layer "F.Cu") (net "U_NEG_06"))
 (segment (start 107.212489 89.53482) (end 106.505382 90.241926) (width 0.03) (layer "F.Cu") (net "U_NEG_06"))
 (segment (start 106.505382 90.241926) (end 101.697056 92.363247) (width 0.03) (layer "F.Cu") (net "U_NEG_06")))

